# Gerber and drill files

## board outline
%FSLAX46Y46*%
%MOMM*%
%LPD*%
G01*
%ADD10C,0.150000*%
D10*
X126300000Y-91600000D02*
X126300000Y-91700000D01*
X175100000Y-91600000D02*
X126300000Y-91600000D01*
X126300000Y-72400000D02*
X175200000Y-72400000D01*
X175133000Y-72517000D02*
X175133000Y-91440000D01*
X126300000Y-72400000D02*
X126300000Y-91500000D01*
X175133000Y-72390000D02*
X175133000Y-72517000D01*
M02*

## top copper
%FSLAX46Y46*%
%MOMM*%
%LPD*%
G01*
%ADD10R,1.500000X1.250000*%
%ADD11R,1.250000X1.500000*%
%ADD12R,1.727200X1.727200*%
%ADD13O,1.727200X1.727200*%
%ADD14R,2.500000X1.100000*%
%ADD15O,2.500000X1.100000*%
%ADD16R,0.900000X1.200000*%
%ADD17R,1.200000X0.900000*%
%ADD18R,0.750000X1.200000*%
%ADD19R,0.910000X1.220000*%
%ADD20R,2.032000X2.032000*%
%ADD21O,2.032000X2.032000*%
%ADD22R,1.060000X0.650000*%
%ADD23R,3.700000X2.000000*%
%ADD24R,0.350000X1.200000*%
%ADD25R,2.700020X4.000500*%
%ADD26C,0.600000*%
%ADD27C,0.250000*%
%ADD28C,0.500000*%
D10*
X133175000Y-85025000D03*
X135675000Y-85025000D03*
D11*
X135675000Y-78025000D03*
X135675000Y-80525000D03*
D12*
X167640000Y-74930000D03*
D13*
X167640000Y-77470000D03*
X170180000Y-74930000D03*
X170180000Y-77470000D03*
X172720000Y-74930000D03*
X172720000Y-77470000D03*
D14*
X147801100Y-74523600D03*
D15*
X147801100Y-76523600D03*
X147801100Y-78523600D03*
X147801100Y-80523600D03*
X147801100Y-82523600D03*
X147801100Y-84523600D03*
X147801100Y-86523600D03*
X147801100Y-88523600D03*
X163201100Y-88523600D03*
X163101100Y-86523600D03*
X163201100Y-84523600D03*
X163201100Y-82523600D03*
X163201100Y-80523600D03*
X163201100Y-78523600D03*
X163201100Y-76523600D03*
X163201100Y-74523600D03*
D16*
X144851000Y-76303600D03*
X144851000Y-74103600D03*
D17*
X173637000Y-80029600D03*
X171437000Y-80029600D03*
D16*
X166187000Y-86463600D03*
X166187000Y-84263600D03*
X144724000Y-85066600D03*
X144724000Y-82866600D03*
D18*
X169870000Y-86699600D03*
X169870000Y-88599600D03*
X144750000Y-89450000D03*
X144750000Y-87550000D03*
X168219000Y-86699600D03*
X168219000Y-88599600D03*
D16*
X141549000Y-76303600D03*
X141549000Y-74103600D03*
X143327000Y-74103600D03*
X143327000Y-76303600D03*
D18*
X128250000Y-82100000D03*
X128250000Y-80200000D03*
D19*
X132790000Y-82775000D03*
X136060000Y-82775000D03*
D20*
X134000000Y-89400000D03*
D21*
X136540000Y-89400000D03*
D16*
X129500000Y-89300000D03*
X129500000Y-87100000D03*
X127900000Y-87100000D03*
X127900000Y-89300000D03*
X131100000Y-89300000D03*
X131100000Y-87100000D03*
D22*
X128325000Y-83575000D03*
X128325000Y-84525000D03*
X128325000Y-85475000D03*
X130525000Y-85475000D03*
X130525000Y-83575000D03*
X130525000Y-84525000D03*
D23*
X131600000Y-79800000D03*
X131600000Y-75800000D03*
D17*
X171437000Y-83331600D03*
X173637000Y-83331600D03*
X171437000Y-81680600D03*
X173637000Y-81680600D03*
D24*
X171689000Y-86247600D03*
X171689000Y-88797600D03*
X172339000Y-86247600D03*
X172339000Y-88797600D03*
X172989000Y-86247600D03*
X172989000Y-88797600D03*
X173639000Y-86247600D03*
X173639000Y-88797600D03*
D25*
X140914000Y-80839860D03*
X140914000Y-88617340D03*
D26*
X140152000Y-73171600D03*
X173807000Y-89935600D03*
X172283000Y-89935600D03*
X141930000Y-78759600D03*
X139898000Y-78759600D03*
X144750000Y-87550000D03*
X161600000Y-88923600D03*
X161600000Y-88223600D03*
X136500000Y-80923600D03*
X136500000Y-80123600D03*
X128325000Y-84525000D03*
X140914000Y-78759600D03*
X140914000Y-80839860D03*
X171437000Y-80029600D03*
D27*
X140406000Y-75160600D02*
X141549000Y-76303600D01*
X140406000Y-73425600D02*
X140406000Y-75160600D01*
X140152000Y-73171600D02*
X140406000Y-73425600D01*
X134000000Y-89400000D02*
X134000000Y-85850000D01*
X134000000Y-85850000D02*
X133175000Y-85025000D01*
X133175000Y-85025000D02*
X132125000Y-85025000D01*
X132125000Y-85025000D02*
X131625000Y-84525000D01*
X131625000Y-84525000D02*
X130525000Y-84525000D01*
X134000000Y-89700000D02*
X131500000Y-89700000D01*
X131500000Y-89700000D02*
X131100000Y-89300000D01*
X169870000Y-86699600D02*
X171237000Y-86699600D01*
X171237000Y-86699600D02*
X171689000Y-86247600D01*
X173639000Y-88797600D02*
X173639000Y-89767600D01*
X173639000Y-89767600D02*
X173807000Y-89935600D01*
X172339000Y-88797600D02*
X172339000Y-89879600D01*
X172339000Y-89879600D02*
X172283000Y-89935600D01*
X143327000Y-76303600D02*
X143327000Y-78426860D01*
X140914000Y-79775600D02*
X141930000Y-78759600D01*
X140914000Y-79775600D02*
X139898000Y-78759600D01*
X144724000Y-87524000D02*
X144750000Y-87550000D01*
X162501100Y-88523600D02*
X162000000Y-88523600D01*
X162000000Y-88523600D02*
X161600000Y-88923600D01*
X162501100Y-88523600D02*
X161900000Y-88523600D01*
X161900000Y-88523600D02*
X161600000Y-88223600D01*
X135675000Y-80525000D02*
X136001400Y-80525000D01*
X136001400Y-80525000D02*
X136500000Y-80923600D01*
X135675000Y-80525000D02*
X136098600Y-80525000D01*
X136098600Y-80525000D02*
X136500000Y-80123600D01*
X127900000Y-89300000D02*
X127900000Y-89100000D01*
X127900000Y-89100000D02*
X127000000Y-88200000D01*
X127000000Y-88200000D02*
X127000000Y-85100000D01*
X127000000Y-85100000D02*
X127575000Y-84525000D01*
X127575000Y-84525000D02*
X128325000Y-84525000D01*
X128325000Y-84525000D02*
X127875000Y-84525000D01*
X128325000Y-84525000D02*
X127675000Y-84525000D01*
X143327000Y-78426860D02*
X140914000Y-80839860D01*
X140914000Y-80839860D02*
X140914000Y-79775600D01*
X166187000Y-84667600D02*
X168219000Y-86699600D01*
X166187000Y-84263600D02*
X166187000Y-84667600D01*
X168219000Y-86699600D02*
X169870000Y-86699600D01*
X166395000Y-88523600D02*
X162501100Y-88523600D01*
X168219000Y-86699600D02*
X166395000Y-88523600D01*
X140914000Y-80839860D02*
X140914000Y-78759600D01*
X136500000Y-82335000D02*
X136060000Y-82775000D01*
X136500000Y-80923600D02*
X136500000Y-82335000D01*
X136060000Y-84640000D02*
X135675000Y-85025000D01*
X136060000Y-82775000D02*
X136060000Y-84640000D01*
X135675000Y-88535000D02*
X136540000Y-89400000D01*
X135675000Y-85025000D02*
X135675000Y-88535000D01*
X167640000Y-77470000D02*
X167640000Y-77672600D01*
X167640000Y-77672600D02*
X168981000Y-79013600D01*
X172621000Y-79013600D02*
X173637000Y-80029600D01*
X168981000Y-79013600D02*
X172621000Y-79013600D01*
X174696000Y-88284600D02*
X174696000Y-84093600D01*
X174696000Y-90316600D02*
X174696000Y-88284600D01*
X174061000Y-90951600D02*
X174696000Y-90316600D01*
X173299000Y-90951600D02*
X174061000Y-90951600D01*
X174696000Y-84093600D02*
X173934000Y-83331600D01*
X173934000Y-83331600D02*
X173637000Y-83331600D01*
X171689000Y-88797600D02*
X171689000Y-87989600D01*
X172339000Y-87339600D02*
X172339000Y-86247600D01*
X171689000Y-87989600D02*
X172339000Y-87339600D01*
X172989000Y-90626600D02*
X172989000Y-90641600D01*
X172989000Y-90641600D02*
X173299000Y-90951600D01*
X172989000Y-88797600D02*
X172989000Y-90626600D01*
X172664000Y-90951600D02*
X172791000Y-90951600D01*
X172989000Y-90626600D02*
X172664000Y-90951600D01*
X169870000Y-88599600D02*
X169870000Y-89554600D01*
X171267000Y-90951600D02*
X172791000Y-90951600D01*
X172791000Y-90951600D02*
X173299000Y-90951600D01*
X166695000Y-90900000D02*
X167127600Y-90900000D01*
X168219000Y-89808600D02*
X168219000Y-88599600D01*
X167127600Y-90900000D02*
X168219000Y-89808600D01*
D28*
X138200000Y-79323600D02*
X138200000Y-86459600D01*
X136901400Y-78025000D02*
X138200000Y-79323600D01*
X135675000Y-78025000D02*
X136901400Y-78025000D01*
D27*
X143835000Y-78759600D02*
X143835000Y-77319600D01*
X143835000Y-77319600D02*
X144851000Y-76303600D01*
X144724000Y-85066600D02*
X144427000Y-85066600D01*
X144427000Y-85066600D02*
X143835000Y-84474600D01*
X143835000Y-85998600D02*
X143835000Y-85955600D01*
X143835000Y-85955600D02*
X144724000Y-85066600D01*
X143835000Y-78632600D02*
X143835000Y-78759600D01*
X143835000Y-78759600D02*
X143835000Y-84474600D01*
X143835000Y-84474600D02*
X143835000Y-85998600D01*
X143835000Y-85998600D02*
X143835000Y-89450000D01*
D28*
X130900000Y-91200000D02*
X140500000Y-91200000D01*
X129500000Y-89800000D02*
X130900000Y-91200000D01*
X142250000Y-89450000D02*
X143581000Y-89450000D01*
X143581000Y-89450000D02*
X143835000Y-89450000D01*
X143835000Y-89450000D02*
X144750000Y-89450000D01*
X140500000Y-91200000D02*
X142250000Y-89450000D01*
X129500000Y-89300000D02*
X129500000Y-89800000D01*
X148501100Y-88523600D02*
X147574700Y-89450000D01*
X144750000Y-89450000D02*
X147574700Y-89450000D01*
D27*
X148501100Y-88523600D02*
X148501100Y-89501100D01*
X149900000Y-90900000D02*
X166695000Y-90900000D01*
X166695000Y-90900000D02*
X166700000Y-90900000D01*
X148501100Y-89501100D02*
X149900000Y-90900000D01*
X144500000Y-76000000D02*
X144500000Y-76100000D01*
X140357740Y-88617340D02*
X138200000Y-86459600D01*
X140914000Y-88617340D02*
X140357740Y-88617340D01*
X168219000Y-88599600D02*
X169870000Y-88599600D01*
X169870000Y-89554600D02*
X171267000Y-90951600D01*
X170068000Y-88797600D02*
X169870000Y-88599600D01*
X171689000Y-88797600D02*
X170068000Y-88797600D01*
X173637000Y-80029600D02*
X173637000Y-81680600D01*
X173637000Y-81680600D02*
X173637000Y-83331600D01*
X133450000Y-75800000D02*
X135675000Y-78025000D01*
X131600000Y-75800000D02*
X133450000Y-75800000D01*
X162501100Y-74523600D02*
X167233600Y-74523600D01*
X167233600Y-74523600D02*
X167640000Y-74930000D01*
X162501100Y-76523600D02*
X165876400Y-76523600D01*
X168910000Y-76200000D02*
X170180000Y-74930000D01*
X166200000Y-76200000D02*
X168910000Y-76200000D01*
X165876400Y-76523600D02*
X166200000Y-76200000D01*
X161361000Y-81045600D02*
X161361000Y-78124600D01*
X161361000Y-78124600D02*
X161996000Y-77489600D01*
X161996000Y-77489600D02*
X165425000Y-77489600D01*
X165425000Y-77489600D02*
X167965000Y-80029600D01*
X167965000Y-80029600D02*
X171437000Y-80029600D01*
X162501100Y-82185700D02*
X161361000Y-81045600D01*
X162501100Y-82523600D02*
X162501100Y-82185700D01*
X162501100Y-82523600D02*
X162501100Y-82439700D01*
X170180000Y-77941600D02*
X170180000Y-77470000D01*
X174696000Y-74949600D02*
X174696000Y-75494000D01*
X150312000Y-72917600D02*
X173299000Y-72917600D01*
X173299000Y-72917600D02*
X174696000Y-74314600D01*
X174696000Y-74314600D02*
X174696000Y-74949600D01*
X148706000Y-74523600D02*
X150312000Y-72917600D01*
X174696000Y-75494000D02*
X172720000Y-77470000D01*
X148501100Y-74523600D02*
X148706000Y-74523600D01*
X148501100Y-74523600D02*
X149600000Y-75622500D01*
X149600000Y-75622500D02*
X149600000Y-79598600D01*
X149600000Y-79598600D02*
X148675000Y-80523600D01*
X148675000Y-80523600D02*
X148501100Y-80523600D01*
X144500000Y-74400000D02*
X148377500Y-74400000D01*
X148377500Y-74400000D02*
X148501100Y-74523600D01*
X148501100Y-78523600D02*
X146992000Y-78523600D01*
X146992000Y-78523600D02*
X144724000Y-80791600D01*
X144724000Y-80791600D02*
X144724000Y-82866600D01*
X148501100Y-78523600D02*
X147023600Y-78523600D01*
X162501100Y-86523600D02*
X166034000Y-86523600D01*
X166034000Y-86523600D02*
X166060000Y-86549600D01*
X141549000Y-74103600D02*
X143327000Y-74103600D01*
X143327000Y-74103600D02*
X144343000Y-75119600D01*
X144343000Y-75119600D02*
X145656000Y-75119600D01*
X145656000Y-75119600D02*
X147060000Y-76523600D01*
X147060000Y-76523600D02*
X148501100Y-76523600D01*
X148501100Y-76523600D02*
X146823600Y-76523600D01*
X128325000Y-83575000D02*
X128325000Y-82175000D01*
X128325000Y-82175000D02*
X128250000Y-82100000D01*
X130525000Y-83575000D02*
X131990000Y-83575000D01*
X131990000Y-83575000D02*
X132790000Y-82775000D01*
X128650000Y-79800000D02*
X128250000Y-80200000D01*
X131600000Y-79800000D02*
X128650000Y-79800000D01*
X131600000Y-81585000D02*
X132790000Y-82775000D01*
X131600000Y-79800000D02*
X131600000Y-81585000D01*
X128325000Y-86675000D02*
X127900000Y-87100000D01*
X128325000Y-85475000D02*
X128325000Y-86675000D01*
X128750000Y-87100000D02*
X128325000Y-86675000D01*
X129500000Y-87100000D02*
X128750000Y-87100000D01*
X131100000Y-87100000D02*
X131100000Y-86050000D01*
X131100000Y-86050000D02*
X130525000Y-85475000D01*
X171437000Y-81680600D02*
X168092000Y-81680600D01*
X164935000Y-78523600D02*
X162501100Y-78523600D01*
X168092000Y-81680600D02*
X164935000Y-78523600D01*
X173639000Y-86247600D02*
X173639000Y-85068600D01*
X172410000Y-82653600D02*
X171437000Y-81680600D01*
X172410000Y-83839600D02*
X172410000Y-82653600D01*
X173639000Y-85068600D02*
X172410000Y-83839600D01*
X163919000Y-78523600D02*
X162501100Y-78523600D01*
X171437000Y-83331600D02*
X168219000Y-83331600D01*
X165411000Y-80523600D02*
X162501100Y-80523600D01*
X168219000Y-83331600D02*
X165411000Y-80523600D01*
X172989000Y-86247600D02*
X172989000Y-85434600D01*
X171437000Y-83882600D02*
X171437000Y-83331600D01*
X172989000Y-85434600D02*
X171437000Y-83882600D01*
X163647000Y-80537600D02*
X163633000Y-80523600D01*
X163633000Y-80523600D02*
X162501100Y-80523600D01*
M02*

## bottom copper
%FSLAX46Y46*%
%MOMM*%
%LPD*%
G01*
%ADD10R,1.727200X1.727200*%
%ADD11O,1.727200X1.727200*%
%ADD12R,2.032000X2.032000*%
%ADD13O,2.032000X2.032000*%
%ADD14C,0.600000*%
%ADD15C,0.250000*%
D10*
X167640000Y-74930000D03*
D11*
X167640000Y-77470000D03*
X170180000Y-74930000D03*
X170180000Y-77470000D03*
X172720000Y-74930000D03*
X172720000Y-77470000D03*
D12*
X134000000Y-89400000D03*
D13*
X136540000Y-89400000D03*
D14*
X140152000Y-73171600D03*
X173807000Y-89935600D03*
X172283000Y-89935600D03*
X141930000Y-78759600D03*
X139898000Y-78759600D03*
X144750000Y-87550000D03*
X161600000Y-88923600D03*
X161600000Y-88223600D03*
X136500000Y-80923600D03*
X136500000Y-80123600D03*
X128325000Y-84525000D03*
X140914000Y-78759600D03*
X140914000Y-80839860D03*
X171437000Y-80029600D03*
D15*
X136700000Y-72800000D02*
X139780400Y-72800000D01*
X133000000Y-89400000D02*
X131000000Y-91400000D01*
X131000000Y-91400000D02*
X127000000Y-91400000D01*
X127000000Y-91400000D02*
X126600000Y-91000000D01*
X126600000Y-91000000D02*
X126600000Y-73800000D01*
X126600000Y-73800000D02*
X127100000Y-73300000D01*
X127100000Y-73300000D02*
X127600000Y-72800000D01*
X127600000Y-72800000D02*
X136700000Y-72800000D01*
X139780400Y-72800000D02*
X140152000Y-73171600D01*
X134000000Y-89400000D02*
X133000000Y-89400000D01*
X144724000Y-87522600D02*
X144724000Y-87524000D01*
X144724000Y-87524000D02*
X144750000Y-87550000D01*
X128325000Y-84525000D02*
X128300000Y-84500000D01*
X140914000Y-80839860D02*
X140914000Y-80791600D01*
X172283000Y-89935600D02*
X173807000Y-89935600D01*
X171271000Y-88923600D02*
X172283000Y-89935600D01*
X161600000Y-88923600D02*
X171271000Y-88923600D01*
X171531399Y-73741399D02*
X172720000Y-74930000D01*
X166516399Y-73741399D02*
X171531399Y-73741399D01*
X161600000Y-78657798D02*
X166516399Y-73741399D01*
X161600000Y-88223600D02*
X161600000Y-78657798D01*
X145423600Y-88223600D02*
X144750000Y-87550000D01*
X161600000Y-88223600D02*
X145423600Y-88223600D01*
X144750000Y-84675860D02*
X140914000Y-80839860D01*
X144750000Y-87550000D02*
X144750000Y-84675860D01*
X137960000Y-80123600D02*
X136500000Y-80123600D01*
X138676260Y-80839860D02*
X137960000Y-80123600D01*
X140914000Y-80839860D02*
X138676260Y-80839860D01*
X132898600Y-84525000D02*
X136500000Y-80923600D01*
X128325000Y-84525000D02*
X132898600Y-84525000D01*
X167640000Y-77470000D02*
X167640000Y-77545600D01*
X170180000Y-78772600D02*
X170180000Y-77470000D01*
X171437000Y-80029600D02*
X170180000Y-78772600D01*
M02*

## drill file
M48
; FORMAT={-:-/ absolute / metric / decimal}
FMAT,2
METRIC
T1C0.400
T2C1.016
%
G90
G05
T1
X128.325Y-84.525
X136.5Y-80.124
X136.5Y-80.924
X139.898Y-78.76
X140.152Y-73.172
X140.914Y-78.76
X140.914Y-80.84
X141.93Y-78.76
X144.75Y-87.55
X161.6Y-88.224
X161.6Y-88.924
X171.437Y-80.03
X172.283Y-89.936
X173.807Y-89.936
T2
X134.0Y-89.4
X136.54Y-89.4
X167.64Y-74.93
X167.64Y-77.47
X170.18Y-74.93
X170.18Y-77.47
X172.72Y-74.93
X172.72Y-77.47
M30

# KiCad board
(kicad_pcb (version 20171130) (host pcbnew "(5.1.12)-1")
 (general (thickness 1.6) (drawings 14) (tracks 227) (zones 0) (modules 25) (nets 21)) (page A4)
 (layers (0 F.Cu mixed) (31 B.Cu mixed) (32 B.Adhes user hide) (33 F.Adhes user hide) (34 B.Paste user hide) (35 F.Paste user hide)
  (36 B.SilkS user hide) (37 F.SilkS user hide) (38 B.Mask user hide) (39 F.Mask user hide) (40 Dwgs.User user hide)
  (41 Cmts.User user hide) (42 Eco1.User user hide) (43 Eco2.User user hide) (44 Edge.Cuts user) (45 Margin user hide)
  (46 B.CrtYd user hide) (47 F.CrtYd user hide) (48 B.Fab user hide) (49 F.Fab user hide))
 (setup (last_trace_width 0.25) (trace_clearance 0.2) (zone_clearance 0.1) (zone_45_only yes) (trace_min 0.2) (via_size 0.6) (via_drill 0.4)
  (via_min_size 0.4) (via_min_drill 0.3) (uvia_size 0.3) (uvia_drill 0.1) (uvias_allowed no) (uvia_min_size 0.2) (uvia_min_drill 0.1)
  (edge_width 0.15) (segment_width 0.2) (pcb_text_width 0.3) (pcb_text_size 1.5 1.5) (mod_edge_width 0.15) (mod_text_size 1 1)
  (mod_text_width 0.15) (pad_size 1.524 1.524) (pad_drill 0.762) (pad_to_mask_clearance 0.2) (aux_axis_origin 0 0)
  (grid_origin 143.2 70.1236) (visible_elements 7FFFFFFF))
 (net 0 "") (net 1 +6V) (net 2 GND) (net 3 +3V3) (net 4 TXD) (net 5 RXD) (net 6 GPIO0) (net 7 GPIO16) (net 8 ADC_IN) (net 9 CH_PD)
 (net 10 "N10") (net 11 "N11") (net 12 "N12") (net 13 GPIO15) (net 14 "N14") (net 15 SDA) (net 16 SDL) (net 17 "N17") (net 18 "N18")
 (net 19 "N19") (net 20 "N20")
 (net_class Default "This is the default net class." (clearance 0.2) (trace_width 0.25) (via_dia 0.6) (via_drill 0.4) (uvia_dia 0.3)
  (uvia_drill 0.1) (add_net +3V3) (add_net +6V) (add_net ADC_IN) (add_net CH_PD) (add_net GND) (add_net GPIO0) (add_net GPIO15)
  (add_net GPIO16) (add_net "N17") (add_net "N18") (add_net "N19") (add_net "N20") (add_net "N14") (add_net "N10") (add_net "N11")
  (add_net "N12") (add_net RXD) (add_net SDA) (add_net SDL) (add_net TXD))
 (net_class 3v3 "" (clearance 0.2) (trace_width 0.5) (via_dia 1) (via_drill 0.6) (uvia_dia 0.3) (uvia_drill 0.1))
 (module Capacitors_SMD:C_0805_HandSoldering (layer F.Cu) (at 134.425 85.025)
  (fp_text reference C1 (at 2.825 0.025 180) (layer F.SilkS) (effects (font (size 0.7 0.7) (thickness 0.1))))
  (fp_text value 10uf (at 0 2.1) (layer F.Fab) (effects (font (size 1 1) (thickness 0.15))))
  (pad 1 smd rect (at -1.25 0) (size 1.5 1.25) (layers F.Cu F.Paste F.Mask) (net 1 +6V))
  (pad 2 smd rect (at 1.25 0) (size 1.5 1.25) (layers F.Cu F.Paste F.Mask) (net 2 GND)))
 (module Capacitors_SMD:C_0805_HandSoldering (layer F.Cu) (at 135.675 79.275 270)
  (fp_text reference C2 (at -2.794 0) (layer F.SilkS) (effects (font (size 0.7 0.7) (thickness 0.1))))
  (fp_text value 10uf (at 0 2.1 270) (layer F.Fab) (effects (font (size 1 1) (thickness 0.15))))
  (pad 1 smd rect (at -1.25 0 270) (size 1.5 1.25) (layers F.Cu F.Paste F.Mask) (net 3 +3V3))
  (pad 2 smd rect (at 1.25 0 270) (size 1.5 1.25) (layers F.Cu F.Paste F.Mask) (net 2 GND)))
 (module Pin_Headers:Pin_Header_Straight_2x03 (layer B.Cu) (at 167.64 74.93 270)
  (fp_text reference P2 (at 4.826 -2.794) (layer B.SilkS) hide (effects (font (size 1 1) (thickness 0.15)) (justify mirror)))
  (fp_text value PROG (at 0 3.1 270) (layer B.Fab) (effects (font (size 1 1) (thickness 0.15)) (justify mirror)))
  (pad 1 thru_hole rect (at 0 0 270) (size 1.7272 1.7272) (drill 1.016) (layers *.Cu *.Mask B.SilkS) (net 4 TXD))
  (pad 2 thru_hole oval (at 2.54 0 270) (size 1.7272 1.7272) (drill 1.016) (layers *.Cu *.Mask B.SilkS) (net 3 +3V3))
  (pad 3 thru_hole oval (at 0 -2.54 270) (size 1.7272 1.7272) (drill 1.016) (layers *.Cu *.Mask B.SilkS) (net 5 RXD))
  (pad 4 thru_hole oval (at 2.54 -2.54 270) (size 1.7272 1.7272) (drill 1.016) (layers *.Cu *.Mask B.SilkS) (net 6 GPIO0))
  (pad 5 thru_hole oval (at 0 -5.08 270) (size 1.7272 1.7272) (drill 1.016) (layers *.Cu *.Mask B.SilkS) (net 2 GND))
  (pad 6 thru_hole oval (at 2.54 -5.08 270) (size 1.7272 1.7272) (drill 1.016) (layers *.Cu *.Mask B.SilkS) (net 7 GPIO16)))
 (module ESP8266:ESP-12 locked (layer F.Cu) (at 148.5011 74.5236)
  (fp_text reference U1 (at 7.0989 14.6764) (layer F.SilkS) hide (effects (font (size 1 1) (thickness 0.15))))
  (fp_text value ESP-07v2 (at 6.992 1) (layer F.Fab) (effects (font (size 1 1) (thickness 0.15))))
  (pad 1 smd rect (at 0 0) (size 2.5 1.1) (drill (offset -0.7 0)) (layers F.Cu F.Paste F.Mask) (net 7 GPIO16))
  (pad 2 smd oval (at 0 2) (size 2.5 1.1) (drill (offset -0.7 0)) (layers F.Cu F.Paste F.Mask) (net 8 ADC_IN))
  (pad 3 smd oval (at 0 4) (size 2.5 1.1) (drill (offset -0.7 0)) (layers F.Cu F.Paste F.Mask) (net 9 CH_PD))
  (pad 4 smd oval (at 0 6) (size 2.5 1.1) (drill (offset -0.7 0)) (layers F.Cu F.Paste F.Mask) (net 7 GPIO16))
  (pad 5 smd oval (at 0 8) (size 2.5 1.1) (drill (offset -0.7 0)) (layers F.Cu F.Paste F.Mask) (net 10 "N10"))
  (pad 6 smd oval (at 0 10) (size 2.5 1.1) (drill (offset -0.7 0)) (layers F.Cu F.Paste F.Mask) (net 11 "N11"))
  (pad 7 smd oval (at 0 12) (size 2.5 1.1) (drill (offset -0.7 0)) (layers F.Cu F.Paste F.Mask) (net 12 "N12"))
  (pad 8 smd oval (at 0 14) (size 2.5 1.1) (drill (offset -0.7 0)) (layers F.Cu F.Paste F.Mask) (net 3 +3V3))
  (pad 9 smd oval (at 14 14) (size 2.5 1.1) (drill (offset 0.7 0)) (layers F.Cu F.Paste F.Mask) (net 2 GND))
  (pad 10 smd oval (at 14 12) (size 2.5 1.1) (drill (offset 0.6 0)) (layers F.Cu F.Paste F.Mask) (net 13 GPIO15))
  (pad 11 smd oval (at 14 10) (size 2.5 1.1) (drill (offset 0.7 0)) (layers F.Cu F.Paste F.Mask) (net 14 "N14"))
  (pad 12 smd oval (at 14 8) (size 2.5 1.1) (drill (offset 0.7 0)) (layers F.Cu F.Paste F.Mask) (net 6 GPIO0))
  (pad 13 smd oval (at 14 6) (size 2.5 1.1) (drill (offset 0.7 0)) (layers F.Cu F.Paste F.Mask) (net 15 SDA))
  (pad 14 smd oval (at 14 4) (size 2.5 1.1) (drill (offset 0.7 0)) (layers F.Cu F.Paste F.Mask) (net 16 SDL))
  (pad 15 smd oval (at 14 2) (size 2.5 1.1) (drill (offset 0.7 0)) (layers F.Cu F.Paste F.Mask) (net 5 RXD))
  (pad 16 smd oval (at 14 0) (size 2.5 1.1) (drill (offset 0.7 0)) (layers F.Cu F.Paste F.Mask) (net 4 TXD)))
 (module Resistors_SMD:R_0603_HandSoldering (layer F.Cu) (at 144.851 75.2036 90)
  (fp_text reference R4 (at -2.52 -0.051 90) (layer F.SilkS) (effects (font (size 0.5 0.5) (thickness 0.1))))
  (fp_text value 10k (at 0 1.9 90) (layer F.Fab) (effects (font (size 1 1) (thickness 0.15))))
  (pad 1 smd rect (at -1.1 0 90) (size 1.2 0.9) (layers F.Cu F.Paste F.Mask) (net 3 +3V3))
  (pad 2 smd rect (at 1.1 0 90) (size 1.2 0.9) (layers F.Cu F.Paste F.Mask) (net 7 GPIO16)))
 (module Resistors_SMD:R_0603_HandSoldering (layer F.Cu) (at 172.537 80.0296 180)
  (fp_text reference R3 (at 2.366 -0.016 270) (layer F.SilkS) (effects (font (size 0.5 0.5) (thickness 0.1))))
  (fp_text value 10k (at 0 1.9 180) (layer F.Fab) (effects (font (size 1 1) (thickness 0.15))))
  (pad 1 smd rect (at -1.1 0 180) (size 1.2 0.9) (layers F.Cu F.Paste F.Mask) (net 3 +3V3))
  (pad 2 smd rect (at 1.1 0 180) (size 1.2 0.9) (layers F.Cu F.Paste F.Mask) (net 6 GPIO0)))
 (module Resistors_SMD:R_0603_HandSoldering (layer F.Cu) (at 166.187 85.3636 90)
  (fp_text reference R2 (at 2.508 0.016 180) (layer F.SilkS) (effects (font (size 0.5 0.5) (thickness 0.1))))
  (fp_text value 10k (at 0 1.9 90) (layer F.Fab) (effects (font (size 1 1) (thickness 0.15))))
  (pad 1 smd rect (at -1.1 0 90) (size 1.2 0.9) (layers F.Cu F.Paste F.Mask) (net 13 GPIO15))
  (pad 2 smd rect (at 1.1 0 90) (size 1.2 0.9) (layers F.Cu F.Paste F.Mask) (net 2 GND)))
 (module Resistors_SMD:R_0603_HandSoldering (layer F.Cu) (at 144.724 83.9666 90)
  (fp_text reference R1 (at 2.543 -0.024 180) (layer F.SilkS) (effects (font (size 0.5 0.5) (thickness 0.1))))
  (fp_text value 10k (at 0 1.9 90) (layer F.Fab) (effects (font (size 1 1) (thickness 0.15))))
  (pad 1 smd rect (at -1.1 0 90) (size 1.2 0.9) (layers F.Cu F.Paste F.Mask) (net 3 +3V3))
  (pad 2 smd rect (at 1.1 0 90) (size 1.2 0.9) (layers F.Cu F.Paste F.Mask) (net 9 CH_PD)))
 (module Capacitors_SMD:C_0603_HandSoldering (layer F.Cu) (at 169.87 87.6496 270)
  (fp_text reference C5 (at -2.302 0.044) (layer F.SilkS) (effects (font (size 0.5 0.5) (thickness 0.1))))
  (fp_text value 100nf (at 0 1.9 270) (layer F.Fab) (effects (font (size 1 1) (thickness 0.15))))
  (pad 1 smd rect (at -0.95 0 270) (size 1.2 0.75) (layers F.Cu F.Paste F.Mask) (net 2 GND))
  (pad 2 smd rect (at 0.95 0 270) (size 1.2 0.75) (layers F.Cu F.Paste F.Mask) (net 3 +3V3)))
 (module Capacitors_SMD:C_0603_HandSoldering (layer F.Cu) (at 144.75 88.5 90)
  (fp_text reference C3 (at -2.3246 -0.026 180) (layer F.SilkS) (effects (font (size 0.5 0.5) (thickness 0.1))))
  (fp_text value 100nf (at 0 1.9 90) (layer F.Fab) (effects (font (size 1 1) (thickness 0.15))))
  (pad 1 smd rect (at -0.95 0 90) (size 1.2 0.75) (layers F.Cu F.Paste F.Mask) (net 3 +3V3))
  (pad 2 smd rect (at 0.95 0 90) (size 1.2 0.75) (layers F.Cu F.Paste F.Mask) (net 2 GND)))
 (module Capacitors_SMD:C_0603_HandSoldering (layer F.Cu) (at 168.219 87.6496 270)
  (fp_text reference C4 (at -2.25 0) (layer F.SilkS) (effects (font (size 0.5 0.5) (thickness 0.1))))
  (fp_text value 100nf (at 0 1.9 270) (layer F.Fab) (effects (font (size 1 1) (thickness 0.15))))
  (pad 1 smd rect (at -0.95 0 270) (size 1.2 0.75) (layers F.Cu F.Paste F.Mask) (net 2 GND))
  (pad 2 smd rect (at 0.95 0 270) (size 1.2 0.75) (layers F.Cu F.Paste F.Mask) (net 3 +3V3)))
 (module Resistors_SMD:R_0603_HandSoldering (layer F.Cu) (at 141.549 75.2036 90)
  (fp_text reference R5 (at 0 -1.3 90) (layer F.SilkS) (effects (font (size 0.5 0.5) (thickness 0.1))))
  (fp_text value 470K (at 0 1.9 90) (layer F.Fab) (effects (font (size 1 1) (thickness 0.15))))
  (pad 1 smd rect (at -1.1 0 90) (size 1.2 0.9) (layers F.Cu F.Paste F.Mask) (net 1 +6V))
  (pad 2 smd rect (at 1.1 0 90) (size 1.2 0.9) (layers F.Cu F.Paste F.Mask) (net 8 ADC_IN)))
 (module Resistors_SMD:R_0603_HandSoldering (layer F.Cu) (at 143.327 75.2036 270)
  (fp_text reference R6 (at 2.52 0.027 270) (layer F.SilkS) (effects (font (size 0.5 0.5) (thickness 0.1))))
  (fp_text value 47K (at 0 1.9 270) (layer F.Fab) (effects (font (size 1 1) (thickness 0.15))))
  (pad 1 smd rect (at -1.1 0 270) (size 1.2 0.9) (layers F.Cu F.Paste F.Mask) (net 8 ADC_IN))
  (pad 2 smd rect (at 1.1 0 270) (size 1.2 0.9) (layers F.Cu F.Paste F.Mask) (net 2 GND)))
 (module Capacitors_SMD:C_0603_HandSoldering (layer F.Cu) (at 128.25 81.15 90)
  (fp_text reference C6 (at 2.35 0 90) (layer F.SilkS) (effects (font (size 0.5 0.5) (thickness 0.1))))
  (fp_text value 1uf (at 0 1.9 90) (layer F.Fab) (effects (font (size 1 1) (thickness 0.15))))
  (pad 1 smd rect (at -0.95 0 90) (size 1.2 0.75) (layers F.Cu F.Paste F.Mask) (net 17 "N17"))
  (pad 2 smd rect (at 0.95 0 90) (size 1.2 0.75) (layers F.Cu F.Paste F.Mask) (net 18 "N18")))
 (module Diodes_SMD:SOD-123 (layer F.Cu) (at 134.425 82.775)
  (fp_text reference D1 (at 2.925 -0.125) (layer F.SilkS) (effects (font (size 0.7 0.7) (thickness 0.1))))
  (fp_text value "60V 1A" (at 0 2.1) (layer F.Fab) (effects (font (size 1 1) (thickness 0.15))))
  (pad 1 smd rect (at -1.635 0) (size 0.91 1.22) (layers F.Cu F.Paste F.Mask) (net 18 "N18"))
  (pad 2 smd rect (at 1.635 0) (size 0.91 1.22) (layers F.Cu F.Paste F.Mask) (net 2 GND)))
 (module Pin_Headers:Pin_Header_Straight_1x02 (layer F.Cu) (at 134 89.4 90)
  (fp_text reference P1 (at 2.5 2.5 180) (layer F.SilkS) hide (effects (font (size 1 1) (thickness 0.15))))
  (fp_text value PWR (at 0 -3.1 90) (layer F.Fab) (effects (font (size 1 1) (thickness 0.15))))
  (pad 1 thru_hole rect (at 0 0 90) (size 2.032 2.032) (drill 1.016) (layers *.Cu *.Mask F.SilkS) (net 1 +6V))
  (pad 2 thru_hole oval (at 0 2.54 90) (size 2.032 2.032) (drill 1.016) (layers *.Cu *.Mask F.SilkS) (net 2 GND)))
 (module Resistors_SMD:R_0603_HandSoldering (layer F.Cu) (at 129.5 88.2 90)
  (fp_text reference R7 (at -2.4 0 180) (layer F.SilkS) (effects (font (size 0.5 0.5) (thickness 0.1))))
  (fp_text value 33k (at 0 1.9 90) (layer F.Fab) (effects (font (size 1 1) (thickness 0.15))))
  (pad 1 smd rect (at -1.1 0 90) (size 1.2 0.9) (layers F.Cu F.Paste F.Mask) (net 3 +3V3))
  (pad 2 smd rect (at 1.1 0 90) (size 1.2 0.9) (layers F.Cu F.Paste F.Mask) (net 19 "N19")))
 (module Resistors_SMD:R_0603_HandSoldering (layer F.Cu) (at 127.9 88.2 270)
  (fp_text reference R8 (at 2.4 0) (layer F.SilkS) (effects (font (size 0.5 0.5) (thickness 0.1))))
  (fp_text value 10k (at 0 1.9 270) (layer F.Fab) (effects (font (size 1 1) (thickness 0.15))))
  (pad 1 smd rect (at -1.1 0 270) (size 1.2 0.9) (layers F.Cu F.Paste F.Mask) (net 19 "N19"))
  (pad 2 smd rect (at 1.1 0 270) (size 1.2 0.9) (layers F.Cu F.Paste F.Mask) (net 2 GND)))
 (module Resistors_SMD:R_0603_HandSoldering (layer F.Cu) (at 131.1 88.2 90)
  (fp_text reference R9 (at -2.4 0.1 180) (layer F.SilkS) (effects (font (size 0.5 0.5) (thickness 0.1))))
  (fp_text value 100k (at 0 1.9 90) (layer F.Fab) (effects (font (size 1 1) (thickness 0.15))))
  (pad 1 smd rect (at -1.1 0 90) (size 1.2 0.9) (layers F.Cu F.Paste F.Mask) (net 1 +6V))
  (pad 2 smd rect (at 1.1 0 90) (size 1.2 0.9) (layers F.Cu F.Paste F.Mask) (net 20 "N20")))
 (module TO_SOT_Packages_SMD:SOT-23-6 (layer F.Cu) (at 129.425 84.525) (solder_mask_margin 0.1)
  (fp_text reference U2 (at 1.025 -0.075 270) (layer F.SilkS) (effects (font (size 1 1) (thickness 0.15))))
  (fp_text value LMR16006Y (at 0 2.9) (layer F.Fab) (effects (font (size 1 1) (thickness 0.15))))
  (pad 1 smd rect (at -1.1 -0.95) (size 1.06 0.65) (layers F.Cu F.Paste F.Mask) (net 17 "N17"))
  (pad 2 smd rect (at -1.1 0) (size 1.06 0.65) (layers F.Cu F.Paste F.Mask) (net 2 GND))
  (pad 3 smd rect (at -1.1 0.95) (size 1.06 0.65) (layers F.Cu F.Paste F.Mask) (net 19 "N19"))
  (pad 4 smd rect (at 1.1 0.95) (size 1.06 0.65) (layers F.Cu F.Paste F.Mask) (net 20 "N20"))
  (pad 6 smd rect (at 1.1 -0.95) (size 1.06 0.65) (layers F.Cu F.Paste F.Mask) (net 18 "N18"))
  (pad 5 smd rect (at 1.1 0) (size 1.06 0.65) (layers F.Cu F.Paste F.Mask) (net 1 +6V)))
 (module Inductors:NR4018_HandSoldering (layer F.Cu) (at 131.6 77.8 90)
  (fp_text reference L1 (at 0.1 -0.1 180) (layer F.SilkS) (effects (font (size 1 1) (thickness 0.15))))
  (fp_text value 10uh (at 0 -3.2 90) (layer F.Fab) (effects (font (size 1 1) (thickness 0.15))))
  (pad 1 smd rect (at -2 0 90) (size 2 3.7) (layers F.Cu F.Paste F.Mask) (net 18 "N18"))
  (pad 2 smd rect (at 2 0 90) (size 2 3.7) (layers F.Cu F.Paste F.Mask) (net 3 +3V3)))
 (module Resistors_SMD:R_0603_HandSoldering (layer F.Cu) (at 172.537 83.3316)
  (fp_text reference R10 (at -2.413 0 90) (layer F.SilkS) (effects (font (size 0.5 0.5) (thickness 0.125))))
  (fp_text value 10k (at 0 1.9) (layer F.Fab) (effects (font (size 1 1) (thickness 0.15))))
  (pad 1 smd rect (at -1.1 0) (size 1.2 0.9) (layers F.Cu F.Paste F.Mask) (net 15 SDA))
  (pad 2 smd rect (at 1.1 0) (size 1.2 0.9) (layers F.Cu F.Paste F.Mask) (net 3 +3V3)))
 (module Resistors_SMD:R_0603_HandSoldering (layer F.Cu) (at 172.537 81.6806)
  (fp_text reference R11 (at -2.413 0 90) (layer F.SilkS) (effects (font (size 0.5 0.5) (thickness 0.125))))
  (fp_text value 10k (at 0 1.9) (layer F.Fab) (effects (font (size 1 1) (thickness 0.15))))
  (pad 1 smd rect (at -1.1 0) (size 1.2 0.9) (layers F.Cu F.Paste F.Mask) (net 16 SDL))
  (pad 2 smd rect (at 1.1 0) (size 1.2 0.9) (layers F.Cu F.Paste F.Mask) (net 3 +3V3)))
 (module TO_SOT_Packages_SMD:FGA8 (layer F.Cu) (at 172.664 87.5226)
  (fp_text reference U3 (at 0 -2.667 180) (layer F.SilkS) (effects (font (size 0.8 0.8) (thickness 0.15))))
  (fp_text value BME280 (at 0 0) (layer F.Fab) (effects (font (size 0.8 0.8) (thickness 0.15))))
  (pad 1 smd rect (at -0.975 -1.275) (size 0.35 1.2) (layers F.Cu F.Paste F.Mask) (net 2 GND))
  (pad 8 smd rect (at -0.975 1.275) (size 0.35 1.2) (layers F.Cu F.Paste F.Mask) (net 3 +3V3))
  (pad 2 smd rect (at -0.325 -1.275) (size 0.35 1.2) (layers F.Cu F.Paste F.Mask) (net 3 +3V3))
  (pad 7 smd rect (at -0.325 1.275) (size 0.35 1.2) (layers F.Cu F.Paste F.Mask) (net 2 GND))
  (pad 3 smd rect (at 0.325 -1.275) (size 0.35 1.2) (layers F.Cu F.Paste F.Mask) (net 15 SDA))
  (pad 6 smd rect (at 0.325 1.275) (size 0.35 1.2) (layers F.Cu F.Paste F.Mask) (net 3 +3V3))
  (pad 4 smd rect (at 0.975 -1.275) (size 0.35 1.2) (layers F.Cu F.Paste F.Mask) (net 16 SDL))
  (pad 5 smd rect (at 0.975 1.275) (size 0.35 1.2) (layers F.Cu F.Paste F.Mask) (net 2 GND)))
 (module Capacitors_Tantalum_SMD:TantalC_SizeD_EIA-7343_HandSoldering (layer F.Cu) (at 140.914 84.7286 90)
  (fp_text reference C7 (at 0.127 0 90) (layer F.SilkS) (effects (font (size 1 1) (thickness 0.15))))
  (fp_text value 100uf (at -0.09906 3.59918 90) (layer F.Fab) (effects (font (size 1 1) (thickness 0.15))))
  (pad 2 smd rect (at 3.88874 0 90) (size 4.0005 2.70002) (layers F.Cu F.Paste F.Mask) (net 2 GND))
  (pad 1 smd rect (at -3.88874 0 90) (size 4.0005 2.70002) (layers F.Cu F.Paste F.Mask) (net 3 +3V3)))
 (gr_line (start 126.3 91.6) (end 126.3 91.7) (angle 90) (layer Edge.Cuts) (width 0.15))
 (gr_line (start 175.1 91.6) (end 126.3 91.6) (angle 90) (layer Edge.Cuts) (width 0.15))
 (gr_line (start 126.3 72.4) (end 175.2 72.4) (angle 90) (layer Edge.Cuts) (width 0.15))
 (gr_line (start 175.133 72.517) (end 175.133 91.44) (angle 90) (layer Edge.Cuts) (width 0.15))
 (gr_line (start 126.3 72.4) (end 126.3 91.5) (angle 90) (layer Edge.Cuts) (width 0.15))
 (gr_line (start 175.133 72.39) (end 175.133 72.517) (angle 90) (layer Edge.Cuts) (width 0.15))
 (segment (start 136.7 72.8) (end 139.7804 72.8) (width 0.25) (layer B.Cu) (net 1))
 (segment (start 133 89.4) (end 131 91.4) (width 0.25) (layer B.Cu) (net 1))
 (segment (start 131 91.4) (end 127 91.4) (width 0.25) (layer B.Cu) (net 1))
 (segment (start 127 91.4) (end 126.6 91) (width 0.25) (layer B.Cu) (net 1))
 (segment (start 126.6 91) (end 126.6 73.8) (width 0.25) (layer B.Cu) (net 1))
 (segment (start 126.6 73.8) (end 127.1 73.3) (width 0.25) (layer B.Cu) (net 1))
 (segment (start 127.1 73.3) (end 127.6 72.8) (width 0.25) (layer B.Cu) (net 1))
 (segment (start 127.6 72.8) (end 136.7 72.8) (width 0.25) (layer B.Cu) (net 1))
 (segment (start 140.406 75.1606) (end 141.549 76.3036) (width 0.25) (layer F.Cu) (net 1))
 (segment (start 140.406 73.4256) (end 140.406 75.1606) (width 0.25) (layer F.Cu) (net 1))
 (segment (start 140.152 73.1716) (end 140.406 73.4256) (width 0.25) (layer F.Cu) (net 1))
 (via (at 140.152 73.1716) (size 0.6) (drill 0.4) (layers F.Cu B.Cu) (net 1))
 (segment (start 139.7804 72.8) (end 140.152 73.1716) (width 0.25) (layer B.Cu) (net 1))
 (segment (start 134 89.4) (end 134 85.85) (width 0.25) (layer F.Cu) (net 1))
 (segment (start 134 85.85) (end 133.175 85.025) (width 0.25) (layer F.Cu) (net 1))
 (segment (start 134 89.4) (end 133 89.4) (width 0.25) (layer B.Cu) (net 1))
 (segment (start 133.175 85.025) (end 132.125 85.025) (width 0.25) (layer F.Cu) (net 1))
 (segment (start 132.125 85.025) (end 131.625 84.525) (width 0.25) (layer F.Cu) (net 1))
 (segment (start 131.625 84.525) (end 130.525 84.525) (width 0.25) (layer F.Cu) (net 1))
 (segment (start 134 89.7) (end 131.5 89.7) (width 0.25) (layer F.Cu) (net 1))
 (segment (start 131.5 89.7) (end 131.1 89.3) (width 0.25) (layer F.Cu) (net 1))
 (segment (start 169.87 86.6996) (end 171.237 86.6996) (width 0.25) (layer F.Cu) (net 2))
 (segment (start 171.237 86.6996) (end 171.689 86.2476) (width 0.25) (layer F.Cu) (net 2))
 (segment (start 173.639 88.7976) (end 173.639 89.7676) (width 0.25) (layer F.Cu) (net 2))
 (via (at 173.807 89.9356) (size 0.6) (drill 0.4) (layers F.Cu B.Cu) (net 2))
 (segment (start 173.639 89.7676) (end 173.807 89.9356) (width 0.25) (layer F.Cu) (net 2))
 (segment (start 172.339 88.7976) (end 172.339 89.8796) (width 0.25) (layer F.Cu) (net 2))
 (via (at 172.283 89.9356) (size 0.6) (drill 0.4) (layers F.Cu B.Cu) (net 2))
 (segment (start 172.339 89.8796) (end 172.283 89.9356) (width 0.25) (layer F.Cu) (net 2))
 (segment (start 143.327 76.3036) (end 143.327 78.42686) (width 0.25) (layer F.Cu) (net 2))
 (segment (start 140.914 79.7756) (end 141.93 78.7596) (width 0.25) (layer F.Cu) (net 2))
 (via (at 141.93 78.7596) (size 0.6) (drill 0.4) (layers F.Cu B.Cu) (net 2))
 (segment (start 140.914 79.7756) (end 139.898 78.7596) (width 0.25) (layer F.Cu) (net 2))
 (via (at 139.898 78.7596) (size 0.6) (drill 0.4) (layers F.Cu B.Cu) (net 2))
 (segment (start 144.724 87.524) (end 144.75 87.55) (width 0.25) (layer F.Cu) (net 2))
 (via (at 144.75 87.55) (size 0.6) (drill 0.4) (layers F.Cu B.Cu) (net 2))
 (segment (start 144.724 87.5226) (end 144.724 87.524) (width 0.25) (layer B.Cu) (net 2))
 (segment (start 144.724 87.524) (end 144.75 87.55) (width 0.25) (layer B.Cu) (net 2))
 (segment (start 162.5011 88.5236) (end 162 88.5236) (width 0.25) (layer F.Cu) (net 2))
 (segment (start 162 88.5236) (end 161.6 88.9236) (width 0.25) (layer F.Cu) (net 2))
 (via (at 161.6 88.9236) (size 0.6) (drill 0.4) (layers F.Cu B.Cu) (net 2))
 (segment (start 162.5011 88.5236) (end 161.9 88.5236) (width 0.25) (layer F.Cu) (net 2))
 (via (at 161.6 88.2236) (size 0.6) (drill 0.4) (layers F.Cu B.Cu) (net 2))
 (segment (start 161.9 88.5236) (end 161.6 88.2236) (width 0.25) (layer F.Cu) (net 2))
 (segment (start 135.675 80.525) (end 136.0014 80.525) (width 0.25) (layer F.Cu) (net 2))
 (segment (start 136.0014 80.525) (end 136.5 80.9236) (width 0.25) (layer F.Cu) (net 2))
 (via (at 136.5 80.9236) (size 0.6) (drill 0.4) (layers F.Cu B.Cu) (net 2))
 (segment (start 135.675 80.525) (end 136.0986 80.525) (width 0.25) (layer F.Cu) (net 2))
 (segment (start 136.0986 80.525) (end 136.5 80.1236) (width 0.25) (layer F.Cu) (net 2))
 (via (at 136.5 80.1236) (size 0.6) (drill 0.4) (layers F.Cu B.Cu) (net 2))
 (via (at 128.325 84.525) (size 0.6) (drill 0.4) (layers F.Cu B.Cu) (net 2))
 (segment (start 128.325 84.525) (end 128.3 84.5) (width 0.25) (layer B.Cu) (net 2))
 (segment (start 127.9 89.3) (end 127.9 89.1) (width 0.25) (layer F.Cu) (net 2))
 (segment (start 127.9 89.1) (end 127 88.2) (width 0.25) (layer F.Cu) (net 2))
 (segment (start 127 88.2) (end 127 85.1) (width 0.25) (layer F.Cu) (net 2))
 (segment (start 127 85.1) (end 127.575 84.525) (width 0.25) (layer F.Cu) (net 2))
 (segment (start 127.575 84.525) (end 128.325 84.525) (width 0.25) (layer F.Cu) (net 2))
 (segment (start 128.325 84.525) (end 127.875 84.525) (width 0.25) (layer F.Cu) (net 2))
 (segment (start 128.325 84.525) (end 127.675 84.525) (width 0.25) (layer F.Cu) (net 2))
 (segment (start 143.327 78.42686) (end 140.914 80.83986) (width 0.25) (layer F.Cu) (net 2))
 (via (at 140.914 78.7596) (size 0.6) (drill 0.4) (layers F.Cu B.Cu) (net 2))
 (segment (start 140.914 80.83986) (end 140.914 79.7756) (width 0.25) (layer F.Cu) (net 2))
 (via (at 140.914 80.83986) (size 0.6) (drill 0.4) (layers F.Cu B.Cu) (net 2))
 (segment (start 140.914 80.83986) (end 140.914 80.7916) (width 0.25) (layer B.Cu) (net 2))
 (segment (start 166.187 84.6676) (end 168.219 86.6996) (width 0.25) (layer F.Cu) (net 2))
 (segment (start 166.187 84.2636) (end 166.187 84.6676) (width 0.25) (layer F.Cu) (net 2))
 (segment (start 168.219 86.6996) (end 169.87 86.6996) (width 0.25) (layer F.Cu) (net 2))
 (segment (start 172.283 89.9356) (end 173.807 89.9356) (width 0.25) (layer B.Cu) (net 2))
 (segment (start 171.271 88.9236) (end 172.283 89.9356) (width 0.25) (layer B.Cu) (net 2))
 (segment (start 161.6 88.9236) (end 171.271 88.9236) (width 0.25) (layer B.Cu) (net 2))
 (segment (start 171.531399 73.741399) (end 172.72 74.93) (width 0.25) (layer B.Cu) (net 2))
 (segment (start 166.516399 73.741399) (end 171.531399 73.741399) (width 0.25) (layer B.Cu) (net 2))
 (segment (start 161.6 78.657798) (end 166.516399 73.741399) (width 0.25) (layer B.Cu) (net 2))
 (segment (start 161.6 88.2236) (end 161.6 78.657798) (width 0.25) (layer B.Cu) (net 2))
 (segment (start 166.395 88.5236) (end 162.5011 88.5236) (width 0.25) (layer F.Cu) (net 2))
 (segment (start 168.219 86.6996) (end 166.395 88.5236) (width 0.25) (layer F.Cu) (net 2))
 (segment (start 145.4236 88.2236) (end 144.75 87.55) (width 0.25) (layer B.Cu) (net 2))
 (segment (start 161.6 88.2236) (end 145.4236 88.2236) (width 0.25) (layer B.Cu) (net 2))
 (segment (start 140.914 80.83986) (end 140.914 78.7596) (width 0.25) (layer F.Cu) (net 2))
 (segment (start 144.75 84.67586) (end 140.914 80.83986) (width 0.25) (layer B.Cu) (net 2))
 (segment (start 144.75 87.55) (end 144.75 84.67586) (width 0.25) (layer B.Cu) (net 2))
 (segment (start 137.96 80.1236) (end 136.5 80.1236) (width 0.25) (layer B.Cu) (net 2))
 (segment (start 138.67626 80.83986) (end 137.96 80.1236) (width 0.25) (layer B.Cu) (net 2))
 (segment (start 140.914 80.83986) (end 138.67626 80.83986) (width 0.25) (layer B.Cu) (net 2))
 (segment (start 136.5 82.335) (end 136.06 82.775) (width 0.25) (layer F.Cu) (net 2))
 (segment (start 136.5 80.9236) (end 136.5 82.335) (width 0.25) (layer F.Cu) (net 2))
 (segment (start 136.06 84.64) (end 135.675 85.025) (width 0.25) (layer F.Cu) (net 2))
 (segment (start 136.06 82.775) (end 136.06 84.64) (width 0.25) (layer F.Cu) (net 2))
 (segment (start 132.8986 84.525) (end 136.5 80.9236) (width 0.25) (layer B.Cu) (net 2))
 (segment (start 128.325 84.525) (end 132.8986 84.525) (width 0.25) (layer B.Cu) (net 2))
 (segment (start 135.675 88.535) (end 136.54 89.4) (width 0.25) (layer F.Cu) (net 2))
 (segment (start 135.675 85.025) (end 135.675 88.535) (width 0.25) (layer F.Cu) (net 2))
 (segment (start 167.64 77.47) (end 167.64 77.6726) (width 0.25) (layer F.Cu) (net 3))
 (segment (start 167.64 77.6726) (end 168.981 79.0136) (width 0.25) (layer F.Cu) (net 3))
 (segment (start 172.621 79.0136) (end 173.637 80.0296) (width 0.25) (layer F.Cu) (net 3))
 (segment (start 168.981 79.0136) (end 172.621 79.0136) (width 0.25) (layer F.Cu) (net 3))
 (segment (start 167.64 77.47) (end 167.64 77.5456) (width 0.25) (layer B.Cu) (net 3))
 (segment (start 174.696 88.2846) (end 174.696 84.0936) (width 0.25) (layer F.Cu) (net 3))
 (segment (start 174.696 90.3166) (end 174.696 88.2846) (width 0.25) (layer F.Cu) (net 3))
 (segment (start 174.061 90.9516) (end 174.696 90.3166) (width 0.25) (layer F.Cu) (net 3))
 (segment (start 173.299 90.9516) (end 174.061 90.9516) (width 0.25) (layer F.Cu) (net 3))
 (segment (start 174.696 84.0936) (end 173.934 83.3316) (width 0.25) (layer F.Cu) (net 3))
 (segment (start 173.934 83.3316) (end 173.637 83.3316) (width 0.25) (layer F.Cu) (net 3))
 (segment (start 171.689 88.7976) (end 171.689 87.9896) (width 0.25) (layer F.Cu) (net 3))
 (segment (start 172.339 87.3396) (end 172.339 86.2476) (width 0.25) (layer F.Cu) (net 3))
 (segment (start 171.689 87.9896) (end 172.339 87.3396) (width 0.25) (layer F.Cu) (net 3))
 (segment (start 172.989 90.6266) (end 172.989 90.6416) (width 0.25) (layer F.Cu) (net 3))
 (segment (start 172.989 90.6416) (end 173.299 90.9516) (width 0.25) (layer F.Cu) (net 3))
 (segment (start 172.989 88.7976) (end 172.989 90.6266) (width 0.25) (layer F.Cu) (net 3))
 (segment (start 172.664 90.9516) (end 172.791 90.9516) (width 0.25) (layer F.Cu) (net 3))
 (segment (start 172.989 90.6266) (end 172.664 90.9516) (width 0.25) (layer F.Cu) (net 3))
 (segment (start 169.87 88.5996) (end 169.87 89.5546) (width 0.25) (layer F.Cu) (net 3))
 (segment (start 171.267 90.9516) (end 172.791 90.9516) (width 0.25) (layer F.Cu) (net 3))
 (segment (start 172.791 90.9516) (end 173.299 90.9516) (width 0.25) (layer F.Cu) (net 3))
 (segment (start 166.695 90.9) (end 167.1276 90.9) (width 0.25) (layer F.Cu) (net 3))
 (segment (start 168.219 89.8086) (end 168.219 88.5996) (width 0.25) (layer F.Cu) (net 3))
 (segment (start 167.1276 90.9) (end 168.219 89.8086) (width 0.25) (layer F.Cu) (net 3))
 (segment (start 138.2 79.3236) (end 138.2 86.4596) (width 0.5) (layer F.Cu) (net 3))
 (segment (start 136.9014 78.025) (end 138.2 79.3236) (width 0.5) (layer F.Cu) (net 3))
 (segment (start 135.675 78.025) (end 136.9014 78.025) (width 0.5) (layer F.Cu) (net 3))
 (segment (start 143.835 78.7596) (end 143.835 77.3196) (width 0.25) (layer F.Cu) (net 3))
 (segment (start 143.835 77.3196) (end 144.851 76.3036) (width 0.25) (layer F.Cu) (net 3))
 (segment (start 144.724 85.0666) (end 144.427 85.0666) (width 0.25) (layer F.Cu) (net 3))
 (segment (start 144.427 85.0666) (end 143.835 84.4746) (width 0.25) (layer F.Cu) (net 3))
 (segment (start 143.835 85.9986) (end 143.835 85.9556) (width 0.25) (layer F.Cu) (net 3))
 (segment (start 143.835 85.9556) (end 144.724 85.0666) (width 0.25) (layer F.Cu) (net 3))
 (segment (start 143.835 78.6326) (end 143.835 78.7596) (width 0.25) (layer F.Cu) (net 3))
 (segment (start 143.835 78.7596) (end 143.835 84.4746) (width 0.25) (layer F.Cu) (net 3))
 (segment (start 143.835 84.4746) (end 143.835 85.9986) (width 0.25) (layer F.Cu) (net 3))
 (segment (start 143.835 85.9986) (end 143.835 89.45) (width 0.25) (layer F.Cu) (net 3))
 (segment (start 130.9 91.2) (end 140.5 91.2) (width 0.5) (layer F.Cu) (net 3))
 (segment (start 129.5 89.8) (end 130.9 91.2) (width 0.5) (layer F.Cu) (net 3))
 (segment (start 142.25 89.45) (end 143.581 89.45) (width 0.5) (layer F.Cu) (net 3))
 (segment (start 143.581 89.45) (end 143.835 89.45) (width 0.5) (layer F.Cu) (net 3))
 (segment (start 143.835 89.45) (end 144.75 89.45) (width 0.5) (layer F.Cu) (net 3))
 (segment (start 140.5 91.2) (end 142.25 89.45) (width 0.5) (layer F.Cu) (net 3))
 (segment (start 129.5 89.3) (end 129.5 89.8) (width 0.5) (layer F.Cu) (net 3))
 (segment (start 148.5011 88.5236) (end 147.5747 89.45) (width 0.5) (layer F.Cu) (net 3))
 (segment (start 144.75 89.45) (end 147.5747 89.45) (width 0.5) (layer F.Cu) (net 3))
 (segment (start 148.5011 88.5236) (end 148.5011 89.5011) (width 0.25) (layer F.Cu) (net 3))
 (segment (start 149.9 90.9) (end 166.695 90.9) (width 0.25) (layer F.Cu) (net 3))
 (segment (start 166.695 90.9) (end 166.7 90.9) (width 0.25) (layer F.Cu) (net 3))
 (segment (start 148.5011 89.5011) (end 149.9 90.9) (width 0.25) (layer F.Cu) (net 3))
 (segment (start 144.5 76) (end 144.5 76.1) (width 0.25) (layer F.Cu) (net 3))
 (segment (start 140.35774 88.61734) (end 138.2 86.4596) (width 0.25) (layer F.Cu) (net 3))
 (segment (start 140.914 88.61734) (end 140.35774 88.61734) (width 0.25) (layer F.Cu) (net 3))
 (segment (start 168.219 88.5996) (end 169.87 88.5996) (width 0.25) (layer F.Cu) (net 3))
 (segment (start 169.87 89.5546) (end 171.267 90.9516) (width 0.25) (layer F.Cu) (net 3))
 (segment (start 170.068 88.7976) (end 169.87 88.5996) (width 0.25) (layer F.Cu) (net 3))
 (segment (start 171.689 88.7976) (end 170.068 88.7976) (width 0.25) (layer F.Cu) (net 3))
 (segment (start 173.637 80.0296) (end 173.637 81.6806) (width 0.25) (layer F.Cu) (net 3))
 (segment (start 173.637 81.6806) (end 173.637 83.3316) (width 0.25) (layer F.Cu) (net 3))
 (segment (start 133.45 75.8) (end 135.675 78.025) (width 0.25) (layer F.Cu) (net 3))
 (segment (start 131.6 75.8) (end 133.45 75.8) (width 0.25) (layer F.Cu) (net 3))
 (segment (start 162.5011 74.5236) (end 167.2336 74.5236) (width 0.25) (layer F.Cu) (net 4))
 (segment (start 167.2336 74.5236) (end 167.64 74.93) (width 0.25) (layer F.Cu) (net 4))
 (segment (start 162.5011 76.5236) (end 165.8764 76.5236) (width 0.25) (layer F.Cu) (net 5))
 (segment (start 168.91 76.2) (end 170.18 74.93) (width 0.25) (layer F.Cu) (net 5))
 (segment (start 166.2 76.2) (end 168.91 76.2) (width 0.25) (layer F.Cu) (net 5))
 (segment (start 165.8764 76.5236) (end 166.2 76.2) (width 0.25) (layer F.Cu) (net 5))
 (via (at 171.437 80.0296) (size 0.6) (drill 0.4) (layers F.Cu B.Cu) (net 6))
 (segment (start 161.361 81.0456) (end 161.361 78.1246) (width 0.25) (layer F.Cu) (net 6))
 (segment (start 161.361 78.1246) (end 161.996 77.4896) (width 0.25) (layer F.Cu) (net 6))
 (segment (start 161.996 77.4896) (end 165.425 77.4896) (width 0.25) (layer F.Cu) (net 6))
 (segment (start 165.425 77.4896) (end 167.965 80.0296) (width 0.25) (layer F.Cu) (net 6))
 (segment (start 167.965 80.0296) (end 171.437 80.0296) (width 0.25) (layer F.Cu) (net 6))
 (segment (start 162.5011 82.1857) (end 161.361 81.0456) (width 0.25) (layer F.Cu) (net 6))
 (segment (start 170.18 78.7726) (end 170.18 77.47) (width 0.25) (layer B.Cu) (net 6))
 (segment (start 171.437 80.0296) (end 170.18 78.7726) (width 0.25) (layer B.Cu) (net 6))
 (segment (start 162.5011 82.5236) (end 162.5011 82.1857) (width 0.25) (layer F.Cu) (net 6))
 (segment (start 162.5011 82.5236) (end 162.5011 82.4397) (width 0.25) (layer F.Cu) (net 6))
 (segment (start 170.18 77.9416) (end 170.18 77.47) (width 0.25) (layer F.Cu) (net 6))
 (segment (start 174.696 74.9496) (end 174.696 75.494) (width 0.25) (layer F.Cu) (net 7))
 (segment (start 150.312 72.9176) (end 173.299 72.9176) (width 0.25) (layer F.Cu) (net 7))
 (segment (start 173.299 72.9176) (end 174.696 74.3146) (width 0.25) (layer F.Cu) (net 7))
 (segment (start 174.696 74.3146) (end 174.696 74.9496) (width 0.25) (layer F.Cu) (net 7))
 (segment (start 148.706 74.5236) (end 150.312 72.9176) (width 0.25) (layer F.Cu) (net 7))
 (segment (start 174.696 75.494) (end 172.72 77.47) (width 0.25) (layer F.Cu) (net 7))
 (segment (start 148.5011 74.5236) (end 148.706 74.5236) (width 0.25) (layer F.Cu) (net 7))
 (segment (start 148.5011 74.5236) (end 149.6 75.6225) (width 0.25) (layer F.Cu) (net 7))
 (segment (start 149.6 75.6225) (end 149.6 79.5986) (width 0.25) (layer F.Cu) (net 7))
 (segment (start 149.6 79.5986) (end 148.675 80.5236) (width 0.25) (layer F.Cu) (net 7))
 (segment (start 148.675 80.5236) (end 148.5011 80.5236) (width 0.25) (layer F.Cu) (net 7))
 (segment (start 144.5 74.4) (end 148.3775 74.4) (width 0.25) (layer F.Cu) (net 7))
 (segment (start 148.3775 74.4) (end 148.5011 74.5236) (width 0.25) (layer F.Cu) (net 7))
 (segment (start 148.5011 78.5236) (end 146.992 78.5236) (width 0.25) (layer F.Cu) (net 9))
 (segment (start 146.992 78.5236) (end 144.724 80.7916) (width 0.25) (layer F.Cu) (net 9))
 (segment (start 144.724 80.7916) (end 144.724 82.8666) (width 0.25) (layer F.Cu) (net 9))
 (segment (start 148.5011 78.5236) (end 147.0236 78.5236) (width 0.25) (layer F.Cu) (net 9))
 (segment (start 162.5011 86.5236) (end 166.034 86.5236) (width 0.25) (layer F.Cu) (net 13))
 (segment (start 166.034 86.5236) (end 166.06 86.5496) (width 0.25) (layer F.Cu) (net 13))
 (segment (start 141.549 74.1036) (end 143.327 74.1036) (width 0.25) (layer F.Cu) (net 8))
 (segment (start 143.327 74.1036) (end 144.343 75.1196) (width 0.25) (layer F.Cu) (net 8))
 (segment (start 144.343 75.1196) (end 145.656 75.1196) (width 0.25) (layer F.Cu) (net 8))
 (segment (start 145.656 75.1196) (end 147.06 76.5236) (width 0.25) (layer F.Cu) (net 8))
 (segment (start 147.06 76.5236) (end 148.5011 76.5236) (width 0.25) (layer F.Cu) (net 8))
 (segment (start 148.5011 76.5236) (end 146.8236 76.5236) (width 0.25) (layer F.Cu) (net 8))
 (segment (start 128.325 83.575) (end 128.325 82.175) (width 0.25) (layer F.Cu) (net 17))
 (segment (start 128.325 82.175) (end 128.25 82.1) (width 0.25) (layer F.Cu) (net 17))
 (segment (start 130.525 83.575) (end 131.99 83.575) (width 0.25) (layer F.Cu) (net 18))
 (segment (start 131.99 83.575) (end 132.79 82.775) (width 0.25) (layer F.Cu) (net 18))
 (segment (start 128.65 79.8) (end 128.25 80.2) (width 0.25) (layer F.Cu) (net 18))
 (segment (start 131.6 79.8) (end 128.65 79.8) (width 0.25) (layer F.Cu) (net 18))
 (segment (start 131.6 81.585) (end 132.79 82.775) (width 0.25) (layer F.Cu) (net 18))
 (segment (start 131.6 79.8) (end 131.6 81.585) (width 0.25) (layer F.Cu) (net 18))
 (segment (start 128.325 86.675) (end 127.9 87.1) (width 0.25) (layer F.Cu) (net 19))
 (segment (start 128.325 85.475) (end 128.325 86.675) (width 0.25) (layer F.Cu) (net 19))
 (segment (start 128.75 87.1) (end 128.325 86.675) (width 0.25) (layer F.Cu) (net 19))
 (segment (start 129.5 87.1) (end 128.75 87.1) (width 0.25) (layer F.Cu) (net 19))
 (segment (start 131.1 87.1) (end 131.1 86.05) (width 0.25) (layer F.Cu) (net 20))
 (segment (start 131.1 86.05) (end 130.525 85.475) (width 0.25) (layer F.Cu) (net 20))
 (segment (start 171.437 81.6806) (end 168.092 81.6806) (width 0.25) (layer F.Cu) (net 16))
 (segment (start 164.935 78.5236) (end 162.5011 78.5236) (width 0.25) (layer F.Cu) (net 16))
 (segment (start 168.092 81.6806) (end 164.935 78.5236) (width 0.25) (layer F.Cu) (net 16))
 (segment (start 173.639 86.2476) (end 173.639 85.0686) (width 0.25) (layer F.Cu) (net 16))
 (segment (start 172.41 82.6536) (end 171.437 81.6806) (width 0.25) (layer F.Cu) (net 16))
 (segment (start 172.41 83.8396) (end 172.41 82.6536) (width 0.25) (layer F.Cu) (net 16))
 (segment (start 173.639 85.0686) (end 172.41 83.8396) (width 0.25) (layer F.Cu) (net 16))
 (segment (start 163.919 78.5236) (end 162.5011 78.5236) (width 0.25) (layer F.Cu) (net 16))
 (segment (start 171.437 83.3316) (end 168.219 83.3316) (width 0.25) (layer F.Cu) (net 15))
 (segment (start 165.411 80.5236) (end 162.5011 80.5236) (width 0.25) (layer F.Cu) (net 15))
 (segment (start 168.219 83.3316) (end 165.411 80.5236) (width 0.25) (layer F.Cu) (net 15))
 (segment (start 172.989 86.2476) (end 172.989 85.4346) (width 0.25) (layer F.Cu) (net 15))
 (segment (start 171.437 83.8826) (end 171.437 83.3316) (width 0.25) (layer F.Cu) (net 15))
 (segment (start 172.989 85.4346) (end 171.437 83.8826) (width 0.25) (layer F.Cu) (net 15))
 (segment (start 163.647 80.5376) (end 163.633 80.5236) (width 0.25) (layer F.Cu) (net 15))
 (segment (start 163.633 80.5236) (end 162.5011 80.5236) (width 0.25) (layer F.Cu) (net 15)))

